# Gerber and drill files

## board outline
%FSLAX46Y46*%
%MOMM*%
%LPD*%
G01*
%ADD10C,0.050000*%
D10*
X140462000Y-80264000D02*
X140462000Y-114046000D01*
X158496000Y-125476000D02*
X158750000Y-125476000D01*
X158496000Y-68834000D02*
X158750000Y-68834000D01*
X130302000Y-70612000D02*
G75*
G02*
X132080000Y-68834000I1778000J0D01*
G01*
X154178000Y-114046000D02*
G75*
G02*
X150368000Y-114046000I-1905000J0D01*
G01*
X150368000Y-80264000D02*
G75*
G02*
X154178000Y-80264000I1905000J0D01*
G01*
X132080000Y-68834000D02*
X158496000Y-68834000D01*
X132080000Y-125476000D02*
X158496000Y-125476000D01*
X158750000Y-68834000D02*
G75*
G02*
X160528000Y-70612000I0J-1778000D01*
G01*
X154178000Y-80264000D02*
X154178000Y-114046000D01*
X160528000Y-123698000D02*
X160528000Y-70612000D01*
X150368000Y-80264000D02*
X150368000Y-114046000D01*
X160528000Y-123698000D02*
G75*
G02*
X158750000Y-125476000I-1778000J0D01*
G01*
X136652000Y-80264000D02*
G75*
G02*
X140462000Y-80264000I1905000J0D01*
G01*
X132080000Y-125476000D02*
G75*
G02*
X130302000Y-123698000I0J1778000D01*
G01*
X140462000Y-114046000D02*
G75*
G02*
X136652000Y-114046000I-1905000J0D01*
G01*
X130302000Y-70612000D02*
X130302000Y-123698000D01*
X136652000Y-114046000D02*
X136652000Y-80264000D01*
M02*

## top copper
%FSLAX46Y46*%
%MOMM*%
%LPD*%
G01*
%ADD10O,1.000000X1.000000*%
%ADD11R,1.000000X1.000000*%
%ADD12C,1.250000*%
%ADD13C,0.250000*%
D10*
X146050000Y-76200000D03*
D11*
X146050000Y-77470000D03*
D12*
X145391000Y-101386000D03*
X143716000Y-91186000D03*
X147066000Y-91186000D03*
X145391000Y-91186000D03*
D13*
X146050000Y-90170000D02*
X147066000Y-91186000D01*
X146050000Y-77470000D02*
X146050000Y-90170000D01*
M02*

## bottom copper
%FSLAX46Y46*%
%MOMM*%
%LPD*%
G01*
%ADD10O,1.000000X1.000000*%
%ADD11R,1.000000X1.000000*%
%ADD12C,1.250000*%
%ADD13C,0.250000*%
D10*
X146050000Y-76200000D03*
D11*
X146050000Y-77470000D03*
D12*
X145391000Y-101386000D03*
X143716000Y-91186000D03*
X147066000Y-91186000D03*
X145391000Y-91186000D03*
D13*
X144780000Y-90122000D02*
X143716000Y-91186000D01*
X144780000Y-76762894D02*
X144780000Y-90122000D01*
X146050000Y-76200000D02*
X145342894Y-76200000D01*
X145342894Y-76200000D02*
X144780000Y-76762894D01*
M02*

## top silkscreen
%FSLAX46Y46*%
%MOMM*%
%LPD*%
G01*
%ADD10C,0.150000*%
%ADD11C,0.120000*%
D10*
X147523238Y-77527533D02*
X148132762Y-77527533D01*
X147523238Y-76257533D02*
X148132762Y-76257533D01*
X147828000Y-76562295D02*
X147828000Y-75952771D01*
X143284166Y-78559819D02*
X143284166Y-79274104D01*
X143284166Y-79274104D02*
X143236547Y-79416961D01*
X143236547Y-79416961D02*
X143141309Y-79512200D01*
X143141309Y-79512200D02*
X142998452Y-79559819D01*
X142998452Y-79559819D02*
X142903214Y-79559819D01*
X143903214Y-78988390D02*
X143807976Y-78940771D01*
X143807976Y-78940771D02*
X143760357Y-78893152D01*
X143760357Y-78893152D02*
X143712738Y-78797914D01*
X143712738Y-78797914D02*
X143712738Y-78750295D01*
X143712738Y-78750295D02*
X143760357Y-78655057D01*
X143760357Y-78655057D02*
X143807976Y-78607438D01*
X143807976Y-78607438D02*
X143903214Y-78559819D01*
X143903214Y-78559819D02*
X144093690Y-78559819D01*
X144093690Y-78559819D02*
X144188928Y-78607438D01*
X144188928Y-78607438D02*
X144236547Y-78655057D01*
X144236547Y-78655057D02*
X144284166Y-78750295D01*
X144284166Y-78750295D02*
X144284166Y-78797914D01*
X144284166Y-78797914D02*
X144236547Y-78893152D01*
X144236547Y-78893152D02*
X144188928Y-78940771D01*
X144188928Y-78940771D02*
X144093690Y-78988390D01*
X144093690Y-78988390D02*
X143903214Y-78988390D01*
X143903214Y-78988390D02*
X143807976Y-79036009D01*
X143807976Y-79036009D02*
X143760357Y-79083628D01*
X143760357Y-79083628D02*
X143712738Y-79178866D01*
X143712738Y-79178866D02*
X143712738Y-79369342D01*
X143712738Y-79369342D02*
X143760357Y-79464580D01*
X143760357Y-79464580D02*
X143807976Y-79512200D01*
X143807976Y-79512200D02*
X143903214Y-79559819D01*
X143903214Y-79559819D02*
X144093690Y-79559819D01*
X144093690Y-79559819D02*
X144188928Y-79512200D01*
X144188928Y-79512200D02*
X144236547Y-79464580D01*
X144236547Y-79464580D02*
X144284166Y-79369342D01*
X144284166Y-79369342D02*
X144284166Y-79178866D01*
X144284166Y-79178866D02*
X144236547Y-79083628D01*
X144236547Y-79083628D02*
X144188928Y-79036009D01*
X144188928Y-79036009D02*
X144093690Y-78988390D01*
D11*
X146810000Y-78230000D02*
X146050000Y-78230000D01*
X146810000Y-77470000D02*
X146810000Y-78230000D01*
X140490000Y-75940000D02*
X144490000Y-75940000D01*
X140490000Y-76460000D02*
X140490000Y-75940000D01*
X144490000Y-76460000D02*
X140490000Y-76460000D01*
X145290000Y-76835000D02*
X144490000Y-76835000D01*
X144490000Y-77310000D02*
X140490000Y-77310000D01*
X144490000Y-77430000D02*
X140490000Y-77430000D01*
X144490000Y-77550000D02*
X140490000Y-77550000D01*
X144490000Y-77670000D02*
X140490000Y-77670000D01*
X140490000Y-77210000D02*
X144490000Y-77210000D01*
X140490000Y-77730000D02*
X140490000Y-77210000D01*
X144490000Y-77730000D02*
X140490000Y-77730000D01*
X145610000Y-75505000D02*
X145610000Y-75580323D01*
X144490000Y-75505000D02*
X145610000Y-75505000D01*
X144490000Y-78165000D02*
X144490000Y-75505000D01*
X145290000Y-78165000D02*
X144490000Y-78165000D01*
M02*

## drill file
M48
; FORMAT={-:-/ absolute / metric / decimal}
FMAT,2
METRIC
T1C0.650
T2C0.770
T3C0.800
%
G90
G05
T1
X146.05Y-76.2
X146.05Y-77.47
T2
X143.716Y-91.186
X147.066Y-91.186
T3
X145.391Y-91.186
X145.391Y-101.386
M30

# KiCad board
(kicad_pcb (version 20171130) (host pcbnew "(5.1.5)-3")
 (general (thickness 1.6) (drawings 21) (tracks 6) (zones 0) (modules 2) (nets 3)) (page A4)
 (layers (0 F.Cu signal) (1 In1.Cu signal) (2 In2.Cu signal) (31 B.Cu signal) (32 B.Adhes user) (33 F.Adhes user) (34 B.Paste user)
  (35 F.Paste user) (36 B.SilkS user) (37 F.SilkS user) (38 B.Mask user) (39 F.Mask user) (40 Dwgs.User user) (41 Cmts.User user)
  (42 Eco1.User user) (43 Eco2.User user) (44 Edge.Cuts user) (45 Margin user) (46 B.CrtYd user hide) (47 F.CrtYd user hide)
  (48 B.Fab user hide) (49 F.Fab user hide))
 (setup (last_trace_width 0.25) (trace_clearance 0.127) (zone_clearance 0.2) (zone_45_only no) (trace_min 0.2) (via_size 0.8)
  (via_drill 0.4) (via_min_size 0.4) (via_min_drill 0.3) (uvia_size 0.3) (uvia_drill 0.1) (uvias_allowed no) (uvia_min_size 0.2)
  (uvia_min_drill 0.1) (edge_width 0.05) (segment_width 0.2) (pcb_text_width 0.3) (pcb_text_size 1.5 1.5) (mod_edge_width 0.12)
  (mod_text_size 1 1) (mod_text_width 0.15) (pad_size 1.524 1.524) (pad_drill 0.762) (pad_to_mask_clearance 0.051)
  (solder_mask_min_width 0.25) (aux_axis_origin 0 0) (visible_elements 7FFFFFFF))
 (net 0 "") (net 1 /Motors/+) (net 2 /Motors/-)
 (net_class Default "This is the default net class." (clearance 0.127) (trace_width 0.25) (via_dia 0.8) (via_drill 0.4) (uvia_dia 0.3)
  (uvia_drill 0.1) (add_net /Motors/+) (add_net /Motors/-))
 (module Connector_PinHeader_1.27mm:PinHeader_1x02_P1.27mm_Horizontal (layer F.Cu) (at 146.05 77.47 180)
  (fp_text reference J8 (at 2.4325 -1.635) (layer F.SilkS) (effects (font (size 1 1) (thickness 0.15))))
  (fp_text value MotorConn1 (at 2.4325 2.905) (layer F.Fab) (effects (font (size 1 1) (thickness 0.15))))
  (fp_line (start -0.76 -0.76) (end 0 -0.76) (layer F.SilkS) (width 0.12))
  (fp_line (start -0.76 0) (end -0.76 -0.76) (layer F.SilkS) (width 0.12))
  (fp_line (start 5.56 1.53) (end 1.56 1.53) (layer F.SilkS) (width 0.12))
  (fp_line (start 5.56 1.01) (end 5.56 1.53) (layer F.SilkS) (width 0.12))
  (fp_line (start 1.56 1.01) (end 5.56 1.01) (layer F.SilkS) (width 0.12))
  (fp_line (start 0.76 0.635) (end 1.56 0.635) (layer F.SilkS) (width 0.12))
  (fp_line (start 1.56 0.16) (end 5.56 0.16) (layer F.SilkS) (width 0.12))
  (fp_line (start 1.56 0.04) (end 5.56 0.04) (layer F.SilkS) (width 0.12))
  (fp_line (start 1.56 -0.08) (end 5.56 -0.08) (layer F.SilkS) (width 0.12))
  (fp_line (start 1.56 -0.2) (end 5.56 -0.2) (layer F.SilkS) (width 0.12))
  (fp_line (start 5.56 0.26) (end 1.56 0.26) (layer F.SilkS) (width 0.12))
  (fp_line (start 5.56 -0.26) (end 5.56 0.26) (layer F.SilkS) (width 0.12))
  (fp_line (start 1.56 -0.26) (end 5.56 -0.26) (layer F.SilkS) (width 0.12))
  (fp_line (start 0.44 1.965) (end 0.44 1.889677) (layer F.SilkS) (width 0.12))
  (fp_line (start 1.56 1.965) (end 0.44 1.965) (layer F.SilkS) (width 0.12))
  (fp_line (start 1.56 -0.695) (end 1.56 1.965) (layer F.SilkS) (width 0.12))
  (fp_line (start 0.76 -0.695) (end 1.56 -0.695) (layer F.SilkS) (width 0.12))
  (pad 2 thru_hole oval (at 0 1.27 180) (size 1 1) (drill 0.65) (layers *.Cu *.Mask) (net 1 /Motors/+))
  (pad 1 thru_hole rect (at 0 0 180) (size 1 1) (drill 0.65) (layers *.Cu *.Mask) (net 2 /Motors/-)))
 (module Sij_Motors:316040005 (layer B.Cu) (at 145.391 91.186)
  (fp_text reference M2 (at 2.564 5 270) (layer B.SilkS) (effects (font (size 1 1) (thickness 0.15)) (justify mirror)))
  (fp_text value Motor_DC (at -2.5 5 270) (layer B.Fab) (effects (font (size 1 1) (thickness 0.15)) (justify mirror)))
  (pad "" thru_hole circle (at 0 10.2) (size 1.25 1.25) (drill 0.8) (layers *.Cu *.Mask))
  (pad 1 thru_hole circle (at -1.675 0) (size 1.25 1.25) (drill 0.77) (layers *.Cu *.Mask) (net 1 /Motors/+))
  (pad 2 thru_hole circle (at 1.675 0) (size 1.25 1.25) (drill 0.77) (layers *.Cu *.Mask) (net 2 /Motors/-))
  (pad "" thru_hole circle (at 0 0) (size 1.25 1.25) (drill 0.8) (layers *.Cu *.Mask)))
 (gr_line (start 140.462 80.264) (end 140.462 114.046) (layer Edge.Cuts) (width 0.05))
 (gr_line (start 158.496 125.476) (end 158.75 125.476) (layer Edge.Cuts) (width 0.05))
 (gr_line (start 158.496 68.834) (end 158.75 68.834) (layer Edge.Cuts) (width 0.05))
 (gr_arc (start 132.08 70.612) (end 132.08 68.834) (angle -90) (layer Edge.Cuts) (width 0.05))
 (gr_arc (start 152.273 114.046) (end 150.368 114.046) (angle -180) (layer Edge.Cuts) (width 0.05))
 (gr_arc (start 152.273 80.264) (end 154.178 80.264) (angle -180) (layer Edge.Cuts) (width 0.05))
 (gr_line (start 132.08 68.834) (end 158.496 68.834) (layer Edge.Cuts) (width 0.05))
 (gr_line (start 132.08 125.476) (end 158.496 125.476) (layer Edge.Cuts) (width 0.05))
 (gr_arc (start 158.75 70.612) (end 160.528 70.612) (angle -90) (layer Edge.Cuts) (width 0.05))
 (gr_line (start 154.178 80.264) (end 154.178 114.046) (layer Edge.Cuts) (width 0.05))
 (gr_line (start 160.528 123.698) (end 160.528 70.612) (layer Edge.Cuts) (width 0.05))
 (gr_line (start 150.368 80.264) (end 150.368 114.046) (layer Edge.Cuts) (width 0.05))
 (gr_arc (start 158.75 123.698) (end 158.75 125.476) (angle -90) (layer Edge.Cuts) (width 0.05))
 (gr_arc (start 138.557 80.264) (end 140.462 80.264) (angle -180) (layer Edge.Cuts) (width 0.05))
 (gr_arc (start 132.08 123.698) (end 130.302 123.698) (angle -90) (layer Edge.Cuts) (width 0.05))
 (gr_arc (start 138.557 114.046) (end 136.652 114.046) (angle -180) (layer Edge.Cuts) (width 0.05))
 (gr_line (start 130.302 70.612) (end 130.302 123.698) (layer Edge.Cuts) (width 0.05))
 (gr_line (start 136.652 114.046) (end 136.652 80.264) (layer Edge.Cuts) (width 0.05))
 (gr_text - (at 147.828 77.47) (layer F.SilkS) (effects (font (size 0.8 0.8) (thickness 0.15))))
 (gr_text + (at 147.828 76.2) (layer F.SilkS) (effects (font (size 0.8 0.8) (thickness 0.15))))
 (segment (start 144.78 90.122) (end 143.716 91.186) (width 0.25) (layer B.Cu) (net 1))
 (segment (start 144.78 76.762894) (end 144.78 90.122) (width 0.25) (layer B.Cu) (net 1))
 (segment (start 146.05 76.2) (end 145.342894 76.2) (width 0.25) (layer B.Cu) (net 1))
 (segment (start 145.342894 76.2) (end 144.78 76.762894) (width 0.25) (layer B.Cu) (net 1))
 (segment (start 146.05 90.17) (end 147.066 91.186) (width 0.25) (layer F.Cu) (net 2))
 (segment (start 146.05 77.47) (end 146.05 90.17) (width 0.25) (layer F.Cu) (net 2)))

